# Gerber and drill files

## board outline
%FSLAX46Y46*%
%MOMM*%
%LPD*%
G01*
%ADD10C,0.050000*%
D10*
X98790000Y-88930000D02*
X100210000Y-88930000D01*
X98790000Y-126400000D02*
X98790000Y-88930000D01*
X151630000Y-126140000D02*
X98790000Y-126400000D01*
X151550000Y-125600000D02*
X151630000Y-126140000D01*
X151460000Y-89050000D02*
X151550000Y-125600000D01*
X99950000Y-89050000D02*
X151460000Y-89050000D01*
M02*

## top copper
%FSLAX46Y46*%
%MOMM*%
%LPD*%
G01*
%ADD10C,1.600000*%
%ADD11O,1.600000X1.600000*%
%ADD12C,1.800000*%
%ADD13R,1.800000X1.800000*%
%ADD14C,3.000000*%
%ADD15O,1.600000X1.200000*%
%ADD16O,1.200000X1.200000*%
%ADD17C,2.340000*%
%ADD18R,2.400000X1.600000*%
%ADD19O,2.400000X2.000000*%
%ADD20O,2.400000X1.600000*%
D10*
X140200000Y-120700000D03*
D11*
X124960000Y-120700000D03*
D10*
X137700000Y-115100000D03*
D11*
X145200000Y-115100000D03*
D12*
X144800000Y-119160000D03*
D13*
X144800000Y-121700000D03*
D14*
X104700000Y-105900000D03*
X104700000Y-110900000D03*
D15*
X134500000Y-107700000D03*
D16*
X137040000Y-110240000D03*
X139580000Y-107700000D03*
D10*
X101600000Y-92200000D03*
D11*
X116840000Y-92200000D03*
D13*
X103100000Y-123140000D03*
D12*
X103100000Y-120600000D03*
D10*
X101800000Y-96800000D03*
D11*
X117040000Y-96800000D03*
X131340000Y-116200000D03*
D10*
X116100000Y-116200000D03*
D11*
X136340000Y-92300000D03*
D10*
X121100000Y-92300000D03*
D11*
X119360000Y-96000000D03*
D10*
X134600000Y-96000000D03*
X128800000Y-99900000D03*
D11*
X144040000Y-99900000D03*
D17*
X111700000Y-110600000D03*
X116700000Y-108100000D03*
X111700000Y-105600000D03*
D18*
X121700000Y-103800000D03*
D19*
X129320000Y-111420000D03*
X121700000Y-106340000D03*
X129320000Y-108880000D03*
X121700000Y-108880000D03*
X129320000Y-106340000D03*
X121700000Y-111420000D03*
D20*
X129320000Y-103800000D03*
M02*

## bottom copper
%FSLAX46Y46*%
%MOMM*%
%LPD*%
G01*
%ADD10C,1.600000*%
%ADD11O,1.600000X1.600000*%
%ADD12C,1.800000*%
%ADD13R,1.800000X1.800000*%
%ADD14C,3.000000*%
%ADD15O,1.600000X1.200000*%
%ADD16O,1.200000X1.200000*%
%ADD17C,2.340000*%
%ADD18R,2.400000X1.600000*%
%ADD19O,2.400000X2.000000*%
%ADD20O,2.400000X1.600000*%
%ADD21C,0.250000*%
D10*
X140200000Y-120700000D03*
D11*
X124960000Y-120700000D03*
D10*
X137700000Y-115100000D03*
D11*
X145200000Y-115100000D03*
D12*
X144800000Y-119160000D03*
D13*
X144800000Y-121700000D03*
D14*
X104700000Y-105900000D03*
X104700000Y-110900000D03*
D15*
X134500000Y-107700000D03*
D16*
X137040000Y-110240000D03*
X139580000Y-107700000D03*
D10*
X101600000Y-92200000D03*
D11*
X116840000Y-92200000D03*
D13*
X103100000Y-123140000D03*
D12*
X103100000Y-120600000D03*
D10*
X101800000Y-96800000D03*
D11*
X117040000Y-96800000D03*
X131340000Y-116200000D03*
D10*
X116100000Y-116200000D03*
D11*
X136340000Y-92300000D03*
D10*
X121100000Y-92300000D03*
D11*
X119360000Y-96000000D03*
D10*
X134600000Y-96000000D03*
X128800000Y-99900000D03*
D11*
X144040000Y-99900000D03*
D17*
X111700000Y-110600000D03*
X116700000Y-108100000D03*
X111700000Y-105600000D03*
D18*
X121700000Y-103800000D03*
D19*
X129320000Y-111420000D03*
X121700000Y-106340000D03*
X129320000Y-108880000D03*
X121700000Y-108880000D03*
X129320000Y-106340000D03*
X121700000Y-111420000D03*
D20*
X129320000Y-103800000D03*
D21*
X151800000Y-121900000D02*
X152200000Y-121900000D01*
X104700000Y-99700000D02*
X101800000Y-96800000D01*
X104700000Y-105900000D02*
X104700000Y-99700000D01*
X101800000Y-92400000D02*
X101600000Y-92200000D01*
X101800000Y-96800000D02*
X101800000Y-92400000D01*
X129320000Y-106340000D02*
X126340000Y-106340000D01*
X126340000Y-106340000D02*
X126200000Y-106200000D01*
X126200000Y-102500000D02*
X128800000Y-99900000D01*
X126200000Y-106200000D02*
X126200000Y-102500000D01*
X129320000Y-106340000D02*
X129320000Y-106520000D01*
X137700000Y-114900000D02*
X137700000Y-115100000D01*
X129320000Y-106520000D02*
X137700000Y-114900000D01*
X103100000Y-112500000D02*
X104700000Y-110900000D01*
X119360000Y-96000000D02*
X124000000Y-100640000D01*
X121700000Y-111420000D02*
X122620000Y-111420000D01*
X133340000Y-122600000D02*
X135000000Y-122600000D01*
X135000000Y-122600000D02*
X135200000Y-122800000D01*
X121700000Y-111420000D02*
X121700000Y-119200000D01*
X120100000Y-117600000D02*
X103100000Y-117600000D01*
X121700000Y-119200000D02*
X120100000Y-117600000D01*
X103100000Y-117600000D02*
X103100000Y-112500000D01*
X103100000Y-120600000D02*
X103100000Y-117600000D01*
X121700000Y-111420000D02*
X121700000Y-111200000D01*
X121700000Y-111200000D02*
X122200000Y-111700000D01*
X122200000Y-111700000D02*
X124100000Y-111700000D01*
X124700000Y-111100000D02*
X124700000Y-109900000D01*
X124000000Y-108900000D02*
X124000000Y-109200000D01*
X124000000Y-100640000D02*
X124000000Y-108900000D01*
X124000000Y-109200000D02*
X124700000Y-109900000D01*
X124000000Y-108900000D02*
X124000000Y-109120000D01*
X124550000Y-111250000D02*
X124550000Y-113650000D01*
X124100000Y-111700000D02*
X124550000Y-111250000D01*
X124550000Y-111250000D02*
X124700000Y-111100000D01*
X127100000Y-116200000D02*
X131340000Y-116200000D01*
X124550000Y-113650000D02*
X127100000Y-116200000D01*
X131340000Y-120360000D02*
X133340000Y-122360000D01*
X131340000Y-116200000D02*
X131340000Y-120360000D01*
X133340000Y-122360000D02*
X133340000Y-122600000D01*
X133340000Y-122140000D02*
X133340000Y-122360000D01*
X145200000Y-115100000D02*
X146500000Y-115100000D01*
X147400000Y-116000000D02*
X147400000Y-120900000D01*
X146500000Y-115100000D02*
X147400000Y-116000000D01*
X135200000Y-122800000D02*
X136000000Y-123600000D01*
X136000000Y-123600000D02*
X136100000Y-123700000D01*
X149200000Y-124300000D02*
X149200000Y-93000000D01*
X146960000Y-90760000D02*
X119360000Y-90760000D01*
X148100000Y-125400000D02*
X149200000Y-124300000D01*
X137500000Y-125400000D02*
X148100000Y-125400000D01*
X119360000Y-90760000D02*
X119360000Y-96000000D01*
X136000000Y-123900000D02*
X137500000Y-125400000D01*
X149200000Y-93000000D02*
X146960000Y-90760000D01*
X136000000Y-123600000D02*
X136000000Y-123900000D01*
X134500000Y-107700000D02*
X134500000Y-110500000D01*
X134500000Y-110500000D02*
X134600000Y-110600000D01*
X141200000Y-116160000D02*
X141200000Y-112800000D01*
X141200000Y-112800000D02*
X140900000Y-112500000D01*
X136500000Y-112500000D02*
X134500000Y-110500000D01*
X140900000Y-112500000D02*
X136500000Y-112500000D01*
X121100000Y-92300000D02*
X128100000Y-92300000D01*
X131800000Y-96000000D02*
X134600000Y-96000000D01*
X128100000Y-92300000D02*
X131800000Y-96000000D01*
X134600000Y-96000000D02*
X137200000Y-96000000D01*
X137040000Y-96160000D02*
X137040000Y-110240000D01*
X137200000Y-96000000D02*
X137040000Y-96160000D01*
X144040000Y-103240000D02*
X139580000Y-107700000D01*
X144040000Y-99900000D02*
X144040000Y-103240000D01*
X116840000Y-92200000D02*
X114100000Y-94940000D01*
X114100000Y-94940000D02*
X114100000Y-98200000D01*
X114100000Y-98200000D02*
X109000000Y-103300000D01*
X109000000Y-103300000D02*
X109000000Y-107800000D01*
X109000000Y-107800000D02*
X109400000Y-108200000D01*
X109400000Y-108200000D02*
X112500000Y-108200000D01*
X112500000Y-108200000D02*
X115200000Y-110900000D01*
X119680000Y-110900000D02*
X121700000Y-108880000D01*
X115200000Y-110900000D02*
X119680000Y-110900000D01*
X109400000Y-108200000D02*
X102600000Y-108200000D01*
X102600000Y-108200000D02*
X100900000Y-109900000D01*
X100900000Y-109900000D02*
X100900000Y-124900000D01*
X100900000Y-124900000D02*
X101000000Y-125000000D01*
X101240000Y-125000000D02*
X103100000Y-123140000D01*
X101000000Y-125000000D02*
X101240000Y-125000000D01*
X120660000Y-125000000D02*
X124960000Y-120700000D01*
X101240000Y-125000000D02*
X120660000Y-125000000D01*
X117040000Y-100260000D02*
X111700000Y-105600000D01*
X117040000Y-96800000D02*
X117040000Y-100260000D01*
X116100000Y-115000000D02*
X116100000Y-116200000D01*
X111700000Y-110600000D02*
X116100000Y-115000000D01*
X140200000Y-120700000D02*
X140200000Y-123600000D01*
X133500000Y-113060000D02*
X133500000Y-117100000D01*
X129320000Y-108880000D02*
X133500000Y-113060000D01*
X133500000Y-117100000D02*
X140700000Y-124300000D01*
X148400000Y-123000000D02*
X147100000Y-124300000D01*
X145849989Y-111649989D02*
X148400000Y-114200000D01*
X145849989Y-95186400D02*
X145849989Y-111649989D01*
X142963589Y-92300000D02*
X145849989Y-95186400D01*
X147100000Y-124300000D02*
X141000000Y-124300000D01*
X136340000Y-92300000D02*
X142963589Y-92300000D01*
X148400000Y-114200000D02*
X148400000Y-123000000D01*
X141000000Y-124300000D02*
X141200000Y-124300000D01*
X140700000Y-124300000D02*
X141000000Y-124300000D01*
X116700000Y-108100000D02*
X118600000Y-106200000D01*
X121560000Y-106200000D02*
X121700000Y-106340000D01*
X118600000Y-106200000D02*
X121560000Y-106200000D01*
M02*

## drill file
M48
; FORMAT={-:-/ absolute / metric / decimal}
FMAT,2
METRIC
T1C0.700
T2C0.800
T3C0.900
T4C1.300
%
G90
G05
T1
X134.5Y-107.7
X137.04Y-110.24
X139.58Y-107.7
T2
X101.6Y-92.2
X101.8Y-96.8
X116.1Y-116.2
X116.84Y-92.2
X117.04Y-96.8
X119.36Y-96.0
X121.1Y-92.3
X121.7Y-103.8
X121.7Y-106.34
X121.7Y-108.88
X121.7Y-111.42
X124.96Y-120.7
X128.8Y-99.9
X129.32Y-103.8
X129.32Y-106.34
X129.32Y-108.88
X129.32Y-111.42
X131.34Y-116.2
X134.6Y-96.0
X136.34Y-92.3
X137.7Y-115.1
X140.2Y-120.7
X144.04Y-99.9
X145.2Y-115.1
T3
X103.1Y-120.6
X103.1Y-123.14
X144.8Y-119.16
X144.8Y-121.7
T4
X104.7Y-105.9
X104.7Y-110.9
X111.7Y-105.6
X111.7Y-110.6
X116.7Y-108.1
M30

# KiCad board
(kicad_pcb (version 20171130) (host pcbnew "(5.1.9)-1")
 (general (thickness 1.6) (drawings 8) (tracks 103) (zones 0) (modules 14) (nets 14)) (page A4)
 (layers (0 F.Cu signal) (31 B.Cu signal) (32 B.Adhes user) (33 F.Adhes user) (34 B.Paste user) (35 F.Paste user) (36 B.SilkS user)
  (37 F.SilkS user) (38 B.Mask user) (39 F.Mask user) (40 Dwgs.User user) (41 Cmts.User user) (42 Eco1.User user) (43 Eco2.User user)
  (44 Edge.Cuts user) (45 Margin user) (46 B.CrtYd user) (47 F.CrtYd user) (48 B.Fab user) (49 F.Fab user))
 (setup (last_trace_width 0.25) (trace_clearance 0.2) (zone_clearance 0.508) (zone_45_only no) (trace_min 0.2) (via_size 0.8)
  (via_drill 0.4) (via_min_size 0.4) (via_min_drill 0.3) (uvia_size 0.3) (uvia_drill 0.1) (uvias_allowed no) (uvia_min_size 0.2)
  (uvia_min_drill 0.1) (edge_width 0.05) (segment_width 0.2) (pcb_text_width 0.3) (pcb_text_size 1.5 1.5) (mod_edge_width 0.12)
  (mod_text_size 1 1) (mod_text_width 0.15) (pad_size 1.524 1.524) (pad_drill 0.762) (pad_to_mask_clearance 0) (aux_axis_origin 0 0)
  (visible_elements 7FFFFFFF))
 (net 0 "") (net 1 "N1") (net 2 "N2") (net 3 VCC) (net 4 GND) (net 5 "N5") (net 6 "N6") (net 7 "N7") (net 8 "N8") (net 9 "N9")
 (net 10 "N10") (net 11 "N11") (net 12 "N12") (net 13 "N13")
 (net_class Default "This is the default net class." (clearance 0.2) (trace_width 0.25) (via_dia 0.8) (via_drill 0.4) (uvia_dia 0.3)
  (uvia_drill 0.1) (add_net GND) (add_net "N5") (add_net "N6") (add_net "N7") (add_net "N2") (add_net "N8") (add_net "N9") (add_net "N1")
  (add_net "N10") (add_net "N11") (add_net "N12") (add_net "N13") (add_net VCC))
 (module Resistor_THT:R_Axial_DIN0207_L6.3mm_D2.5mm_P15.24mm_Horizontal (layer F.Cu) (at 140.2 120.7 180)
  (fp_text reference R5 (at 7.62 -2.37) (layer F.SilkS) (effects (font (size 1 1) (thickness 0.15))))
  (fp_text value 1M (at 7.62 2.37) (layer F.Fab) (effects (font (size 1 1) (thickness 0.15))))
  (pad 1 thru_hole circle (at 0 0 180) (size 1.6 1.6) (drill 0.8) (layers *.Cu *.Mask) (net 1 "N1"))
  (pad 2 thru_hole oval (at 15.24 0 180) (size 1.6 1.6) (drill 0.8) (layers *.Cu *.Mask) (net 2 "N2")))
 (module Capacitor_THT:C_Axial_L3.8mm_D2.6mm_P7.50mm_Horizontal (layer F.Cu) (at 137.7 115.1)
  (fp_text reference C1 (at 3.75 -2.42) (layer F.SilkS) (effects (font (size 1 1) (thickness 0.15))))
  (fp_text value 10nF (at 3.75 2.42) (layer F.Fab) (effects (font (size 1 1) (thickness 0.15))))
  (pad 1 thru_hole circle (at 0 0) (size 1.6 1.6) (drill 0.8) (layers *.Cu *.Mask) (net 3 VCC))
  (pad 2 thru_hole oval (at 7.5 0) (size 1.6 1.6) (drill 0.8) (layers *.Cu *.Mask) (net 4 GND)))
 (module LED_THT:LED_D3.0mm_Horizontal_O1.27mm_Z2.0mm (layer F.Cu) (at 144.8 121.7 90)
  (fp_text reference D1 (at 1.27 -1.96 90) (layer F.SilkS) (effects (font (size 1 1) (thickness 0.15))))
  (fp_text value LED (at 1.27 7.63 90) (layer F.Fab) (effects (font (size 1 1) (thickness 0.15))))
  (pad 2 thru_hole circle (at 2.54 0 90) (size 1.8 1.8) (drill 0.9) (layers *.Cu *.Mask) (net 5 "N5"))
  (pad 1 thru_hole rect (at 0 0 90) (size 1.8 1.8) (drill 0.9) (layers *.Cu *.Mask) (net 4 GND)))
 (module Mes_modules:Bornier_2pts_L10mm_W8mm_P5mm (layer F.Cu) (at 104.7 105.9 270)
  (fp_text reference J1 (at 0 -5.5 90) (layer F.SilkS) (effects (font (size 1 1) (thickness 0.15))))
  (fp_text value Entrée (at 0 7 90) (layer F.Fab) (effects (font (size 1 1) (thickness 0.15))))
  (pad 1 thru_hole circle (at 0 0 270) (size 3 3) (drill 1.3) (layers *.Cu *.Mask) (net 3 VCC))
  (pad 2 thru_hole circle (at 5 0 270) (size 3 3) (drill 1.3) (layers *.Cu *.Mask) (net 4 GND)))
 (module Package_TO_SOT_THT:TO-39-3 (layer F.Cu) (at 134.5 107.7)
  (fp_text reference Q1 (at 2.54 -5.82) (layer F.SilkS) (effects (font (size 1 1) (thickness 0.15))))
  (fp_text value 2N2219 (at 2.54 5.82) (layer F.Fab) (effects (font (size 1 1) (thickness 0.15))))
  (pad 1 thru_hole oval (at 0 0) (size 1.6 1.2) (drill 0.7) (layers *.Cu *.Mask) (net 5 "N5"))
  (pad 2 thru_hole oval (at 2.54 2.54) (size 1.2 1.2) (drill 0.7) (layers *.Cu *.Mask) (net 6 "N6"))
  (pad 3 thru_hole oval (at 5.08 0) (size 1.2 1.2) (drill 0.7) (layers *.Cu *.Mask) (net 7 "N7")))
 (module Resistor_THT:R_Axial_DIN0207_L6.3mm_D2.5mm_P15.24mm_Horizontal (layer F.Cu) (at 101.6 92.2)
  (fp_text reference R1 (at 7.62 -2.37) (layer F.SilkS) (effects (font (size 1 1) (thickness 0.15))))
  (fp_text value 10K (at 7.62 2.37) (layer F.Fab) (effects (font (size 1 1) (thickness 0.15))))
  (pad 1 thru_hole circle (at 0 0) (size 1.6 1.6) (drill 0.8) (layers *.Cu *.Mask) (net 3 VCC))
  (pad 2 thru_hole oval (at 15.24 0) (size 1.6 1.6) (drill 0.8) (layers *.Cu *.Mask) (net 2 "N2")))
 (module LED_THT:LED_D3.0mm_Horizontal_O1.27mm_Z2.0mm (layer F.Cu) (at 103.1 123.14 90)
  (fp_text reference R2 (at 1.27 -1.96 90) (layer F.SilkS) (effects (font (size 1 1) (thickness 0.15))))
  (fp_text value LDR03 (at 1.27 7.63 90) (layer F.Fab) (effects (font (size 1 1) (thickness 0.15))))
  (pad 1 thru_hole rect (at 0 0 90) (size 1.8 1.8) (drill 0.9) (layers *.Cu *.Mask) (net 2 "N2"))
  (pad 2 thru_hole circle (at 2.54 0 90) (size 1.8 1.8) (drill 0.9) (layers *.Cu *.Mask) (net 4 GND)))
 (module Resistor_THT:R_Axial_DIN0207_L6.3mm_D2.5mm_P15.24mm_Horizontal (layer F.Cu) (at 101.8 96.8)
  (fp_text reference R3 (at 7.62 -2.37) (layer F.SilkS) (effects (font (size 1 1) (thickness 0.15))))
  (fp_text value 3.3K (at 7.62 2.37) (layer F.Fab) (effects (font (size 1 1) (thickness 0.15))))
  (pad 1 thru_hole circle (at 0 0) (size 1.6 1.6) (drill 0.8) (layers *.Cu *.Mask) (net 3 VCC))
  (pad 2 thru_hole oval (at 15.24 0) (size 1.6 1.6) (drill 0.8) (layers *.Cu *.Mask) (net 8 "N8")))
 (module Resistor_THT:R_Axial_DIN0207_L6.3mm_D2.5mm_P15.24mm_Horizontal (layer F.Cu) (at 116.1 116.2)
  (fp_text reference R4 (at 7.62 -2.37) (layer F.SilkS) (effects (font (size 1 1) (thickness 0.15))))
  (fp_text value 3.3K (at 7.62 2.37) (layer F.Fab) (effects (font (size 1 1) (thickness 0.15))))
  (pad 2 thru_hole oval (at 15.24 0) (size 1.6 1.6) (drill 0.8) (layers *.Cu *.Mask) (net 4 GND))
  (pad 1 thru_hole circle (at 0 0) (size 1.6 1.6) (drill 0.8) (layers *.Cu *.Mask) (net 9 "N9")))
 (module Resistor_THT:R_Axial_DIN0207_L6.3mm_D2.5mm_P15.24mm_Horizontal (layer F.Cu) (at 121.1 92.3)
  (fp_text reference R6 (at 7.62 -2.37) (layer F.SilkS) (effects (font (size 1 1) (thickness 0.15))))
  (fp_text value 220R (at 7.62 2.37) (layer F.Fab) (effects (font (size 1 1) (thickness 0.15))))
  (pad 2 thru_hole oval (at 15.24 0) (size 1.6 1.6) (drill 0.8) (layers *.Cu *.Mask) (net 1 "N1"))
  (pad 1 thru_hole circle (at 0 0) (size 1.6 1.6) (drill 0.8) (layers *.Cu *.Mask) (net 6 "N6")))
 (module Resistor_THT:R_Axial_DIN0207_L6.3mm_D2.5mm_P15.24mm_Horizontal (layer F.Cu) (at 134.6 96 180)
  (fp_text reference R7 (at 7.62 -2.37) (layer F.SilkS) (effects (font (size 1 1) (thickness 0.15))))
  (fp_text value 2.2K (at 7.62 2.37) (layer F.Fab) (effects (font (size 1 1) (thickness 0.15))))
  (pad 2 thru_hole oval (at 15.24 0 180) (size 1.6 1.6) (drill 0.8) (layers *.Cu *.Mask) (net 4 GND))
  (pad 1 thru_hole circle (at 0 0 180) (size 1.6 1.6) (drill 0.8) (layers *.Cu *.Mask) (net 6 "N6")))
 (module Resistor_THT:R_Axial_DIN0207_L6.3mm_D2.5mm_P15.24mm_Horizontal (layer F.Cu) (at 128.8 99.9)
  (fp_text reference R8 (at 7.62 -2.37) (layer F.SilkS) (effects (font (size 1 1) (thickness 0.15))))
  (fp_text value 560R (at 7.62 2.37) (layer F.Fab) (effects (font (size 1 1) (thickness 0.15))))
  (pad 1 thru_hole circle (at 0 0) (size 1.6 1.6) (drill 0.8) (layers *.Cu *.Mask) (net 3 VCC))
  (pad 2 thru_hole oval (at 15.24 0) (size 1.6 1.6) (drill 0.8) (layers *.Cu *.Mask) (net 7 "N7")))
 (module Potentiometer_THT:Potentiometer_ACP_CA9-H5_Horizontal (layer F.Cu) (at 111.7 105.6)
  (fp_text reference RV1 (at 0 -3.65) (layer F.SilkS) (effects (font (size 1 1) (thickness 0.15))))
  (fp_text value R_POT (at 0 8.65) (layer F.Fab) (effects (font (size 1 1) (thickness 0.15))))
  (pad 3 thru_hole circle (at 0 5) (size 2.34 2.34) (drill 1.3) (layers *.Cu *.Mask) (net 9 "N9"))
  (pad 2 thru_hole circle (at 5 2.5) (size 2.34 2.34) (drill 1.3) (layers *.Cu *.Mask) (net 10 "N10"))
  (pad 1 thru_hole circle (at 0 0) (size 2.34 2.34) (drill 1.3) (layers *.Cu *.Mask) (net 8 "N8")))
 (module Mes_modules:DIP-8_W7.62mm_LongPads (layer F.Cu) (at 121.7 103.8)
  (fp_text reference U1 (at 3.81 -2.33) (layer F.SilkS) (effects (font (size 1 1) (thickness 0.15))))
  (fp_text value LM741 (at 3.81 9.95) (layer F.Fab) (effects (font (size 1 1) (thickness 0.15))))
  (pad 1 thru_hole rect (at 0 0) (size 2.4 1.6) (drill 0.8) (layers *.Cu *.Mask) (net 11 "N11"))
  (pad 5 thru_hole oval (at 7.62 7.62) (size 2.4 2) (drill 0.8) (layers *.Cu *.Mask) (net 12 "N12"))
  (pad 2 thru_hole oval (at 0 2.54) (size 2.4 2) (drill 0.8) (layers *.Cu *.Mask) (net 10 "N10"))
  (pad 6 thru_hole oval (at 7.62 5.08) (size 2.4 2) (drill 0.8) (layers *.Cu *.Mask) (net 1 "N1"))
  (pad 3 thru_hole oval (at 0 5.08) (size 2.4 2) (drill 0.8) (layers *.Cu *.Mask) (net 2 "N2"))
  (pad 7 thru_hole oval (at 7.62 2.54) (size 2.4 2) (drill 0.8) (layers *.Cu *.Mask) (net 3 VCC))
  (pad 4 thru_hole oval (at 0 7.62) (size 2.4 2) (drill 0.8) (layers *.Cu *.Mask) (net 4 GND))
  (pad 8 thru_hole oval (at 7.62 0) (size 2.4 1.6) (drill 0.8) (layers *.Cu *.Mask) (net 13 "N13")))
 (gr_line (start 98.79 88.93) (end 100.21 88.93) (layer Edge.Cuts) (width 0.05))
 (gr_line (start 98.79 126.4) (end 98.79 88.93) (layer Edge.Cuts) (width 0.05))
 (gr_line (start 151.63 126.14) (end 98.79 126.4) (layer Edge.Cuts) (width 0.05))
 (gr_line (start 151.55 125.6) (end 151.63 126.14) (layer Edge.Cuts) (width 0.05))
 (gr_line (start 151.46 89.05) (end 151.55 125.6) (layer Edge.Cuts) (width 0.05))
 (gr_line (start 99.95 89.05) (end 151.46 89.05) (layer Edge.Cuts) (width 0.05))
 (segment (start 151.8 121.9) (end 152.2 121.9) (width 0.25) (layer B.Cu) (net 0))
 (segment (start 104.7 99.7) (end 101.8 96.8) (width 0.25) (layer B.Cu) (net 3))
 (segment (start 104.7 105.9) (end 104.7 99.7) (width 0.25) (layer B.Cu) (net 3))
 (segment (start 101.8 92.4) (end 101.6 92.2) (width 0.25) (layer B.Cu) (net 3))
 (segment (start 101.8 96.8) (end 101.8 92.4) (width 0.25) (layer B.Cu) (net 3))
 (segment (start 129.32 106.34) (end 126.34 106.34) (width 0.25) (layer B.Cu) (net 3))
 (segment (start 126.34 106.34) (end 126.2 106.2) (width 0.25) (layer B.Cu) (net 3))
 (segment (start 126.2 102.5) (end 128.8 99.9) (width 0.25) (layer B.Cu) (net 3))
 (segment (start 126.2 106.2) (end 126.2 102.5) (width 0.25) (layer B.Cu) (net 3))
 (segment (start 129.32 106.34) (end 129.32 106.52) (width 0.25) (layer B.Cu) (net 3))
 (segment (start 137.7 114.9) (end 137.7 115.1) (width 0.25) (layer B.Cu) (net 3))
 (segment (start 129.32 106.52) (end 137.7 114.9) (width 0.25) (layer B.Cu) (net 3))
 (segment (start 103.1 112.5) (end 104.7 110.9) (width 0.25) (layer B.Cu) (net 4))
 (segment (start 119.36 96) (end 124 100.64) (width 0.25) (layer B.Cu) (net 4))
 (segment (start 121.7 111.42) (end 122.62 111.42) (width 0.25) (layer B.Cu) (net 4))
 (segment (start 133.34 122.6) (end 135 122.6) (width 0.25) (layer B.Cu) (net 4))
 (segment (start 135 122.6) (end 135.2 122.8) (width 0.25) (layer B.Cu) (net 4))
 (segment (start 121.7 111.42) (end 121.7 119.2) (width 0.25) (layer B.Cu) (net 4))
 (segment (start 120.1 117.6) (end 103.1 117.6) (width 0.25) (layer B.Cu) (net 4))
 (segment (start 121.7 119.2) (end 120.1 117.6) (width 0.25) (layer B.Cu) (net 4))
 (segment (start 103.1 117.6) (end 103.1 112.5) (width 0.25) (layer B.Cu) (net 4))
 (segment (start 103.1 120.6) (end 103.1 117.6) (width 0.25) (layer B.Cu) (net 4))
 (segment (start 121.7 111.42) (end 121.7 111.2) (width 0.25) (layer B.Cu) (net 4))
 (segment (start 121.7 111.2) (end 122.2 111.7) (width 0.25) (layer B.Cu) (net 4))
 (segment (start 122.2 111.7) (end 124.1 111.7) (width 0.25) (layer B.Cu) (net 4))
 (segment (start 124.7 111.1) (end 124.7 109.9) (width 0.25) (layer B.Cu) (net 4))
 (segment (start 124 108.9) (end 124 109.2) (width 0.25) (layer B.Cu) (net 4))
 (segment (start 124 100.64) (end 124 108.9) (width 0.25) (layer B.Cu) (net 4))
 (segment (start 124 109.2) (end 124.7 109.9) (width 0.25) (layer B.Cu) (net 4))
 (segment (start 124 108.9) (end 124 109.12) (width 0.25) (layer B.Cu) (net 4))
 (segment (start 124.55 111.25) (end 124.55 113.65) (width 0.25) (layer B.Cu) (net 4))
 (segment (start 124.1 111.7) (end 124.55 111.25) (width 0.25) (layer B.Cu) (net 4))
 (segment (start 124.55 111.25) (end 124.7 111.1) (width 0.25) (layer B.Cu) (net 4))
 (segment (start 127.1 116.2) (end 131.34 116.2) (width 0.25) (layer B.Cu) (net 4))
 (segment (start 124.55 113.65) (end 127.1 116.2) (width 0.25) (layer B.Cu) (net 4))
 (segment (start 131.34 120.36) (end 133.34 122.36) (width 0.25) (layer B.Cu) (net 4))
 (segment (start 131.34 116.2) (end 131.34 120.36) (width 0.25) (layer B.Cu) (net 4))
 (segment (start 133.34 122.36) (end 133.34 122.6) (width 0.25) (layer B.Cu) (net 4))
 (segment (start 133.34 122.14) (end 133.34 122.36) (width 0.25) (layer B.Cu) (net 4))
 (segment (start 145.2 115.1) (end 146.5 115.1) (width 0.25) (layer B.Cu) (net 4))
 (segment (start 147.4 116) (end 147.4 120.9) (width 0.25) (layer B.Cu) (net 4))
 (segment (start 146.5 115.1) (end 147.4 116) (width 0.25) (layer B.Cu) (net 4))
 (segment (start 135.2 122.8) (end 136 123.6) (width 0.25) (layer B.Cu) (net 4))
 (segment (start 136 123.6) (end 136.1 123.7) (width 0.25) (layer B.Cu) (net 4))
 (segment (start 149.2 124.3) (end 149.2 93) (width 0.25) (layer B.Cu) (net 4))
 (segment (start 146.96 90.76) (end 119.36 90.76) (width 0.25) (layer B.Cu) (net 4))
 (segment (start 148.1 125.4) (end 149.2 124.3) (width 0.25) (layer B.Cu) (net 4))
 (segment (start 137.5 125.4) (end 148.1 125.4) (width 0.25) (layer B.Cu) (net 4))
 (segment (start 119.36 90.76) (end 119.36 96) (width 0.25) (layer B.Cu) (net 4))
 (segment (start 136 123.9) (end 137.5 125.4) (width 0.25) (layer B.Cu) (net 4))
 (segment (start 149.2 93) (end 146.96 90.76) (width 0.25) (layer B.Cu) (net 4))
 (segment (start 136 123.6) (end 136 123.9) (width 0.25) (layer B.Cu) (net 4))
 (segment (start 134.5 107.7) (end 134.5 110.5) (width 0.25) (layer B.Cu) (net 5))
 (segment (start 134.5 110.5) (end 134.6 110.6) (width 0.25) (layer B.Cu) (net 5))
 (segment (start 141.2 116.16) (end 141.2 112.8) (width 0.25) (layer B.Cu) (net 5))
 (segment (start 141.2 112.8) (end 140.9 112.5) (width 0.25) (layer B.Cu) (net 5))
 (segment (start 136.5 112.5) (end 134.5 110.5) (width 0.25) (layer B.Cu) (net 5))
 (segment (start 140.9 112.5) (end 136.5 112.5) (width 0.25) (layer B.Cu) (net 5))
 (segment (start 121.1 92.3) (end 128.1 92.3) (width 0.25) (layer B.Cu) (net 6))
 (segment (start 131.8 96) (end 134.6 96) (width 0.25) (layer B.Cu) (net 6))
 (segment (start 128.1 92.3) (end 131.8 96) (width 0.25) (layer B.Cu) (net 6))
 (segment (start 134.6 96) (end 137.2 96) (width 0.25) (layer B.Cu) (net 6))
 (segment (start 137.04 96.16) (end 137.04 110.24) (width 0.25) (layer B.Cu) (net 6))
 (segment (start 137.2 96) (end 137.04 96.16) (width 0.25) (layer B.Cu) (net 6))
 (segment (start 144.04 103.24) (end 139.58 107.7) (width 0.25) (layer B.Cu) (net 7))
 (segment (start 144.04 99.9) (end 144.04 103.24) (width 0.25) (layer B.Cu) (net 7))
 (segment (start 116.84 92.2) (end 114.1 94.94) (width 0.25) (layer B.Cu) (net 2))
 (segment (start 114.1 94.94) (end 114.1 98.2) (width 0.25) (layer B.Cu) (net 2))
 (segment (start 114.1 98.2) (end 109 103.3) (width 0.25) (layer B.Cu) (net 2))
 (segment (start 109 103.3) (end 109 107.8) (width 0.25) (layer B.Cu) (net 2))
 (segment (start 109 107.8) (end 109.4 108.2) (width 0.25) (layer B.Cu) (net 2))
 (segment (start 109.4 108.2) (end 112.5 108.2) (width 0.25) (layer B.Cu) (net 2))
 (segment (start 112.5 108.2) (end 115.2 110.9) (width 0.25) (layer B.Cu) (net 2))
 (segment (start 119.68 110.9) (end 121.7 108.88) (width 0.25) (layer B.Cu) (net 2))
 (segment (start 115.2 110.9) (end 119.68 110.9) (width 0.25) (layer B.Cu) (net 2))
 (segment (start 109.4 108.2) (end 102.6 108.2) (width 0.25) (layer B.Cu) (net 2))
 (segment (start 102.6 108.2) (end 100.9 109.9) (width 0.25) (layer B.Cu) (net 2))
 (segment (start 100.9 109.9) (end 100.9 124.9) (width 0.25) (layer B.Cu) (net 2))
 (segment (start 100.9 124.9) (end 101 125) (width 0.25) (layer B.Cu) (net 2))
 (segment (start 101.24 125) (end 103.1 123.14) (width 0.25) (layer B.Cu) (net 2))
 (segment (start 101 125) (end 101.24 125) (width 0.25) (layer B.Cu) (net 2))
 (segment (start 120.66 125) (end 124.96 120.7) (width 0.25) (layer B.Cu) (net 2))
 (segment (start 101.24 125) (end 120.66 125) (width 0.25) (layer B.Cu) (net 2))
 (segment (start 117.04 100.26) (end 111.7 105.6) (width 0.25) (layer B.Cu) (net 8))
 (segment (start 117.04 96.8) (end 117.04 100.26) (width 0.25) (layer B.Cu) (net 8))
 (segment (start 116.1 115) (end 116.1 116.2) (width 0.25) (layer B.Cu) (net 9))
 (segment (start 111.7 110.6) (end 116.1 115) (width 0.25) (layer B.Cu) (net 9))
 (segment (start 140.2 120.7) (end 140.2 123.6) (width 0.25) (layer B.Cu) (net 1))
 (segment (start 133.5 113.06) (end 133.5 117.1) (width 0.25) (layer B.Cu) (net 1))
 (segment (start 129.32 108.88) (end 133.5 113.06) (width 0.25) (layer B.Cu) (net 1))
 (segment (start 133.5 117.1) (end 140.7 124.3) (width 0.25) (layer B.Cu) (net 1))
 (segment (start 148.4 123) (end 147.1 124.3) (width 0.25) (layer B.Cu) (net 1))
 (segment (start 145.849989 111.649989) (end 148.4 114.2) (width 0.25) (layer B.Cu) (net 1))
 (segment (start 145.849989 95.1864) (end 145.849989 111.649989) (width 0.25) (layer B.Cu) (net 1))
 (segment (start 142.963589 92.3) (end 145.849989 95.1864) (width 0.25) (layer B.Cu) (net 1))
 (segment (start 147.1 124.3) (end 141 124.3) (width 0.25) (layer B.Cu) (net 1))
 (segment (start 136.34 92.3) (end 142.963589 92.3) (width 0.25) (layer B.Cu) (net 1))
 (segment (start 148.4 114.2) (end 148.4 123) (width 0.25) (layer B.Cu) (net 1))
 (segment (start 141 124.3) (end 141.2 124.3) (width 0.25) (layer B.Cu) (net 1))
 (segment (start 140.7 124.3) (end 141 124.3) (width 0.25) (layer B.Cu) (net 1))
 (segment (start 116.7 108.1) (end 118.6 106.2) (width 0.25) (layer B.Cu) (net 10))
 (segment (start 121.56 106.2) (end 121.7 106.34) (width 0.25) (layer B.Cu) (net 10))
 (segment (start 118.6 106.2) (end 121.56 106.2) (width 0.25) (layer B.Cu) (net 10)))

